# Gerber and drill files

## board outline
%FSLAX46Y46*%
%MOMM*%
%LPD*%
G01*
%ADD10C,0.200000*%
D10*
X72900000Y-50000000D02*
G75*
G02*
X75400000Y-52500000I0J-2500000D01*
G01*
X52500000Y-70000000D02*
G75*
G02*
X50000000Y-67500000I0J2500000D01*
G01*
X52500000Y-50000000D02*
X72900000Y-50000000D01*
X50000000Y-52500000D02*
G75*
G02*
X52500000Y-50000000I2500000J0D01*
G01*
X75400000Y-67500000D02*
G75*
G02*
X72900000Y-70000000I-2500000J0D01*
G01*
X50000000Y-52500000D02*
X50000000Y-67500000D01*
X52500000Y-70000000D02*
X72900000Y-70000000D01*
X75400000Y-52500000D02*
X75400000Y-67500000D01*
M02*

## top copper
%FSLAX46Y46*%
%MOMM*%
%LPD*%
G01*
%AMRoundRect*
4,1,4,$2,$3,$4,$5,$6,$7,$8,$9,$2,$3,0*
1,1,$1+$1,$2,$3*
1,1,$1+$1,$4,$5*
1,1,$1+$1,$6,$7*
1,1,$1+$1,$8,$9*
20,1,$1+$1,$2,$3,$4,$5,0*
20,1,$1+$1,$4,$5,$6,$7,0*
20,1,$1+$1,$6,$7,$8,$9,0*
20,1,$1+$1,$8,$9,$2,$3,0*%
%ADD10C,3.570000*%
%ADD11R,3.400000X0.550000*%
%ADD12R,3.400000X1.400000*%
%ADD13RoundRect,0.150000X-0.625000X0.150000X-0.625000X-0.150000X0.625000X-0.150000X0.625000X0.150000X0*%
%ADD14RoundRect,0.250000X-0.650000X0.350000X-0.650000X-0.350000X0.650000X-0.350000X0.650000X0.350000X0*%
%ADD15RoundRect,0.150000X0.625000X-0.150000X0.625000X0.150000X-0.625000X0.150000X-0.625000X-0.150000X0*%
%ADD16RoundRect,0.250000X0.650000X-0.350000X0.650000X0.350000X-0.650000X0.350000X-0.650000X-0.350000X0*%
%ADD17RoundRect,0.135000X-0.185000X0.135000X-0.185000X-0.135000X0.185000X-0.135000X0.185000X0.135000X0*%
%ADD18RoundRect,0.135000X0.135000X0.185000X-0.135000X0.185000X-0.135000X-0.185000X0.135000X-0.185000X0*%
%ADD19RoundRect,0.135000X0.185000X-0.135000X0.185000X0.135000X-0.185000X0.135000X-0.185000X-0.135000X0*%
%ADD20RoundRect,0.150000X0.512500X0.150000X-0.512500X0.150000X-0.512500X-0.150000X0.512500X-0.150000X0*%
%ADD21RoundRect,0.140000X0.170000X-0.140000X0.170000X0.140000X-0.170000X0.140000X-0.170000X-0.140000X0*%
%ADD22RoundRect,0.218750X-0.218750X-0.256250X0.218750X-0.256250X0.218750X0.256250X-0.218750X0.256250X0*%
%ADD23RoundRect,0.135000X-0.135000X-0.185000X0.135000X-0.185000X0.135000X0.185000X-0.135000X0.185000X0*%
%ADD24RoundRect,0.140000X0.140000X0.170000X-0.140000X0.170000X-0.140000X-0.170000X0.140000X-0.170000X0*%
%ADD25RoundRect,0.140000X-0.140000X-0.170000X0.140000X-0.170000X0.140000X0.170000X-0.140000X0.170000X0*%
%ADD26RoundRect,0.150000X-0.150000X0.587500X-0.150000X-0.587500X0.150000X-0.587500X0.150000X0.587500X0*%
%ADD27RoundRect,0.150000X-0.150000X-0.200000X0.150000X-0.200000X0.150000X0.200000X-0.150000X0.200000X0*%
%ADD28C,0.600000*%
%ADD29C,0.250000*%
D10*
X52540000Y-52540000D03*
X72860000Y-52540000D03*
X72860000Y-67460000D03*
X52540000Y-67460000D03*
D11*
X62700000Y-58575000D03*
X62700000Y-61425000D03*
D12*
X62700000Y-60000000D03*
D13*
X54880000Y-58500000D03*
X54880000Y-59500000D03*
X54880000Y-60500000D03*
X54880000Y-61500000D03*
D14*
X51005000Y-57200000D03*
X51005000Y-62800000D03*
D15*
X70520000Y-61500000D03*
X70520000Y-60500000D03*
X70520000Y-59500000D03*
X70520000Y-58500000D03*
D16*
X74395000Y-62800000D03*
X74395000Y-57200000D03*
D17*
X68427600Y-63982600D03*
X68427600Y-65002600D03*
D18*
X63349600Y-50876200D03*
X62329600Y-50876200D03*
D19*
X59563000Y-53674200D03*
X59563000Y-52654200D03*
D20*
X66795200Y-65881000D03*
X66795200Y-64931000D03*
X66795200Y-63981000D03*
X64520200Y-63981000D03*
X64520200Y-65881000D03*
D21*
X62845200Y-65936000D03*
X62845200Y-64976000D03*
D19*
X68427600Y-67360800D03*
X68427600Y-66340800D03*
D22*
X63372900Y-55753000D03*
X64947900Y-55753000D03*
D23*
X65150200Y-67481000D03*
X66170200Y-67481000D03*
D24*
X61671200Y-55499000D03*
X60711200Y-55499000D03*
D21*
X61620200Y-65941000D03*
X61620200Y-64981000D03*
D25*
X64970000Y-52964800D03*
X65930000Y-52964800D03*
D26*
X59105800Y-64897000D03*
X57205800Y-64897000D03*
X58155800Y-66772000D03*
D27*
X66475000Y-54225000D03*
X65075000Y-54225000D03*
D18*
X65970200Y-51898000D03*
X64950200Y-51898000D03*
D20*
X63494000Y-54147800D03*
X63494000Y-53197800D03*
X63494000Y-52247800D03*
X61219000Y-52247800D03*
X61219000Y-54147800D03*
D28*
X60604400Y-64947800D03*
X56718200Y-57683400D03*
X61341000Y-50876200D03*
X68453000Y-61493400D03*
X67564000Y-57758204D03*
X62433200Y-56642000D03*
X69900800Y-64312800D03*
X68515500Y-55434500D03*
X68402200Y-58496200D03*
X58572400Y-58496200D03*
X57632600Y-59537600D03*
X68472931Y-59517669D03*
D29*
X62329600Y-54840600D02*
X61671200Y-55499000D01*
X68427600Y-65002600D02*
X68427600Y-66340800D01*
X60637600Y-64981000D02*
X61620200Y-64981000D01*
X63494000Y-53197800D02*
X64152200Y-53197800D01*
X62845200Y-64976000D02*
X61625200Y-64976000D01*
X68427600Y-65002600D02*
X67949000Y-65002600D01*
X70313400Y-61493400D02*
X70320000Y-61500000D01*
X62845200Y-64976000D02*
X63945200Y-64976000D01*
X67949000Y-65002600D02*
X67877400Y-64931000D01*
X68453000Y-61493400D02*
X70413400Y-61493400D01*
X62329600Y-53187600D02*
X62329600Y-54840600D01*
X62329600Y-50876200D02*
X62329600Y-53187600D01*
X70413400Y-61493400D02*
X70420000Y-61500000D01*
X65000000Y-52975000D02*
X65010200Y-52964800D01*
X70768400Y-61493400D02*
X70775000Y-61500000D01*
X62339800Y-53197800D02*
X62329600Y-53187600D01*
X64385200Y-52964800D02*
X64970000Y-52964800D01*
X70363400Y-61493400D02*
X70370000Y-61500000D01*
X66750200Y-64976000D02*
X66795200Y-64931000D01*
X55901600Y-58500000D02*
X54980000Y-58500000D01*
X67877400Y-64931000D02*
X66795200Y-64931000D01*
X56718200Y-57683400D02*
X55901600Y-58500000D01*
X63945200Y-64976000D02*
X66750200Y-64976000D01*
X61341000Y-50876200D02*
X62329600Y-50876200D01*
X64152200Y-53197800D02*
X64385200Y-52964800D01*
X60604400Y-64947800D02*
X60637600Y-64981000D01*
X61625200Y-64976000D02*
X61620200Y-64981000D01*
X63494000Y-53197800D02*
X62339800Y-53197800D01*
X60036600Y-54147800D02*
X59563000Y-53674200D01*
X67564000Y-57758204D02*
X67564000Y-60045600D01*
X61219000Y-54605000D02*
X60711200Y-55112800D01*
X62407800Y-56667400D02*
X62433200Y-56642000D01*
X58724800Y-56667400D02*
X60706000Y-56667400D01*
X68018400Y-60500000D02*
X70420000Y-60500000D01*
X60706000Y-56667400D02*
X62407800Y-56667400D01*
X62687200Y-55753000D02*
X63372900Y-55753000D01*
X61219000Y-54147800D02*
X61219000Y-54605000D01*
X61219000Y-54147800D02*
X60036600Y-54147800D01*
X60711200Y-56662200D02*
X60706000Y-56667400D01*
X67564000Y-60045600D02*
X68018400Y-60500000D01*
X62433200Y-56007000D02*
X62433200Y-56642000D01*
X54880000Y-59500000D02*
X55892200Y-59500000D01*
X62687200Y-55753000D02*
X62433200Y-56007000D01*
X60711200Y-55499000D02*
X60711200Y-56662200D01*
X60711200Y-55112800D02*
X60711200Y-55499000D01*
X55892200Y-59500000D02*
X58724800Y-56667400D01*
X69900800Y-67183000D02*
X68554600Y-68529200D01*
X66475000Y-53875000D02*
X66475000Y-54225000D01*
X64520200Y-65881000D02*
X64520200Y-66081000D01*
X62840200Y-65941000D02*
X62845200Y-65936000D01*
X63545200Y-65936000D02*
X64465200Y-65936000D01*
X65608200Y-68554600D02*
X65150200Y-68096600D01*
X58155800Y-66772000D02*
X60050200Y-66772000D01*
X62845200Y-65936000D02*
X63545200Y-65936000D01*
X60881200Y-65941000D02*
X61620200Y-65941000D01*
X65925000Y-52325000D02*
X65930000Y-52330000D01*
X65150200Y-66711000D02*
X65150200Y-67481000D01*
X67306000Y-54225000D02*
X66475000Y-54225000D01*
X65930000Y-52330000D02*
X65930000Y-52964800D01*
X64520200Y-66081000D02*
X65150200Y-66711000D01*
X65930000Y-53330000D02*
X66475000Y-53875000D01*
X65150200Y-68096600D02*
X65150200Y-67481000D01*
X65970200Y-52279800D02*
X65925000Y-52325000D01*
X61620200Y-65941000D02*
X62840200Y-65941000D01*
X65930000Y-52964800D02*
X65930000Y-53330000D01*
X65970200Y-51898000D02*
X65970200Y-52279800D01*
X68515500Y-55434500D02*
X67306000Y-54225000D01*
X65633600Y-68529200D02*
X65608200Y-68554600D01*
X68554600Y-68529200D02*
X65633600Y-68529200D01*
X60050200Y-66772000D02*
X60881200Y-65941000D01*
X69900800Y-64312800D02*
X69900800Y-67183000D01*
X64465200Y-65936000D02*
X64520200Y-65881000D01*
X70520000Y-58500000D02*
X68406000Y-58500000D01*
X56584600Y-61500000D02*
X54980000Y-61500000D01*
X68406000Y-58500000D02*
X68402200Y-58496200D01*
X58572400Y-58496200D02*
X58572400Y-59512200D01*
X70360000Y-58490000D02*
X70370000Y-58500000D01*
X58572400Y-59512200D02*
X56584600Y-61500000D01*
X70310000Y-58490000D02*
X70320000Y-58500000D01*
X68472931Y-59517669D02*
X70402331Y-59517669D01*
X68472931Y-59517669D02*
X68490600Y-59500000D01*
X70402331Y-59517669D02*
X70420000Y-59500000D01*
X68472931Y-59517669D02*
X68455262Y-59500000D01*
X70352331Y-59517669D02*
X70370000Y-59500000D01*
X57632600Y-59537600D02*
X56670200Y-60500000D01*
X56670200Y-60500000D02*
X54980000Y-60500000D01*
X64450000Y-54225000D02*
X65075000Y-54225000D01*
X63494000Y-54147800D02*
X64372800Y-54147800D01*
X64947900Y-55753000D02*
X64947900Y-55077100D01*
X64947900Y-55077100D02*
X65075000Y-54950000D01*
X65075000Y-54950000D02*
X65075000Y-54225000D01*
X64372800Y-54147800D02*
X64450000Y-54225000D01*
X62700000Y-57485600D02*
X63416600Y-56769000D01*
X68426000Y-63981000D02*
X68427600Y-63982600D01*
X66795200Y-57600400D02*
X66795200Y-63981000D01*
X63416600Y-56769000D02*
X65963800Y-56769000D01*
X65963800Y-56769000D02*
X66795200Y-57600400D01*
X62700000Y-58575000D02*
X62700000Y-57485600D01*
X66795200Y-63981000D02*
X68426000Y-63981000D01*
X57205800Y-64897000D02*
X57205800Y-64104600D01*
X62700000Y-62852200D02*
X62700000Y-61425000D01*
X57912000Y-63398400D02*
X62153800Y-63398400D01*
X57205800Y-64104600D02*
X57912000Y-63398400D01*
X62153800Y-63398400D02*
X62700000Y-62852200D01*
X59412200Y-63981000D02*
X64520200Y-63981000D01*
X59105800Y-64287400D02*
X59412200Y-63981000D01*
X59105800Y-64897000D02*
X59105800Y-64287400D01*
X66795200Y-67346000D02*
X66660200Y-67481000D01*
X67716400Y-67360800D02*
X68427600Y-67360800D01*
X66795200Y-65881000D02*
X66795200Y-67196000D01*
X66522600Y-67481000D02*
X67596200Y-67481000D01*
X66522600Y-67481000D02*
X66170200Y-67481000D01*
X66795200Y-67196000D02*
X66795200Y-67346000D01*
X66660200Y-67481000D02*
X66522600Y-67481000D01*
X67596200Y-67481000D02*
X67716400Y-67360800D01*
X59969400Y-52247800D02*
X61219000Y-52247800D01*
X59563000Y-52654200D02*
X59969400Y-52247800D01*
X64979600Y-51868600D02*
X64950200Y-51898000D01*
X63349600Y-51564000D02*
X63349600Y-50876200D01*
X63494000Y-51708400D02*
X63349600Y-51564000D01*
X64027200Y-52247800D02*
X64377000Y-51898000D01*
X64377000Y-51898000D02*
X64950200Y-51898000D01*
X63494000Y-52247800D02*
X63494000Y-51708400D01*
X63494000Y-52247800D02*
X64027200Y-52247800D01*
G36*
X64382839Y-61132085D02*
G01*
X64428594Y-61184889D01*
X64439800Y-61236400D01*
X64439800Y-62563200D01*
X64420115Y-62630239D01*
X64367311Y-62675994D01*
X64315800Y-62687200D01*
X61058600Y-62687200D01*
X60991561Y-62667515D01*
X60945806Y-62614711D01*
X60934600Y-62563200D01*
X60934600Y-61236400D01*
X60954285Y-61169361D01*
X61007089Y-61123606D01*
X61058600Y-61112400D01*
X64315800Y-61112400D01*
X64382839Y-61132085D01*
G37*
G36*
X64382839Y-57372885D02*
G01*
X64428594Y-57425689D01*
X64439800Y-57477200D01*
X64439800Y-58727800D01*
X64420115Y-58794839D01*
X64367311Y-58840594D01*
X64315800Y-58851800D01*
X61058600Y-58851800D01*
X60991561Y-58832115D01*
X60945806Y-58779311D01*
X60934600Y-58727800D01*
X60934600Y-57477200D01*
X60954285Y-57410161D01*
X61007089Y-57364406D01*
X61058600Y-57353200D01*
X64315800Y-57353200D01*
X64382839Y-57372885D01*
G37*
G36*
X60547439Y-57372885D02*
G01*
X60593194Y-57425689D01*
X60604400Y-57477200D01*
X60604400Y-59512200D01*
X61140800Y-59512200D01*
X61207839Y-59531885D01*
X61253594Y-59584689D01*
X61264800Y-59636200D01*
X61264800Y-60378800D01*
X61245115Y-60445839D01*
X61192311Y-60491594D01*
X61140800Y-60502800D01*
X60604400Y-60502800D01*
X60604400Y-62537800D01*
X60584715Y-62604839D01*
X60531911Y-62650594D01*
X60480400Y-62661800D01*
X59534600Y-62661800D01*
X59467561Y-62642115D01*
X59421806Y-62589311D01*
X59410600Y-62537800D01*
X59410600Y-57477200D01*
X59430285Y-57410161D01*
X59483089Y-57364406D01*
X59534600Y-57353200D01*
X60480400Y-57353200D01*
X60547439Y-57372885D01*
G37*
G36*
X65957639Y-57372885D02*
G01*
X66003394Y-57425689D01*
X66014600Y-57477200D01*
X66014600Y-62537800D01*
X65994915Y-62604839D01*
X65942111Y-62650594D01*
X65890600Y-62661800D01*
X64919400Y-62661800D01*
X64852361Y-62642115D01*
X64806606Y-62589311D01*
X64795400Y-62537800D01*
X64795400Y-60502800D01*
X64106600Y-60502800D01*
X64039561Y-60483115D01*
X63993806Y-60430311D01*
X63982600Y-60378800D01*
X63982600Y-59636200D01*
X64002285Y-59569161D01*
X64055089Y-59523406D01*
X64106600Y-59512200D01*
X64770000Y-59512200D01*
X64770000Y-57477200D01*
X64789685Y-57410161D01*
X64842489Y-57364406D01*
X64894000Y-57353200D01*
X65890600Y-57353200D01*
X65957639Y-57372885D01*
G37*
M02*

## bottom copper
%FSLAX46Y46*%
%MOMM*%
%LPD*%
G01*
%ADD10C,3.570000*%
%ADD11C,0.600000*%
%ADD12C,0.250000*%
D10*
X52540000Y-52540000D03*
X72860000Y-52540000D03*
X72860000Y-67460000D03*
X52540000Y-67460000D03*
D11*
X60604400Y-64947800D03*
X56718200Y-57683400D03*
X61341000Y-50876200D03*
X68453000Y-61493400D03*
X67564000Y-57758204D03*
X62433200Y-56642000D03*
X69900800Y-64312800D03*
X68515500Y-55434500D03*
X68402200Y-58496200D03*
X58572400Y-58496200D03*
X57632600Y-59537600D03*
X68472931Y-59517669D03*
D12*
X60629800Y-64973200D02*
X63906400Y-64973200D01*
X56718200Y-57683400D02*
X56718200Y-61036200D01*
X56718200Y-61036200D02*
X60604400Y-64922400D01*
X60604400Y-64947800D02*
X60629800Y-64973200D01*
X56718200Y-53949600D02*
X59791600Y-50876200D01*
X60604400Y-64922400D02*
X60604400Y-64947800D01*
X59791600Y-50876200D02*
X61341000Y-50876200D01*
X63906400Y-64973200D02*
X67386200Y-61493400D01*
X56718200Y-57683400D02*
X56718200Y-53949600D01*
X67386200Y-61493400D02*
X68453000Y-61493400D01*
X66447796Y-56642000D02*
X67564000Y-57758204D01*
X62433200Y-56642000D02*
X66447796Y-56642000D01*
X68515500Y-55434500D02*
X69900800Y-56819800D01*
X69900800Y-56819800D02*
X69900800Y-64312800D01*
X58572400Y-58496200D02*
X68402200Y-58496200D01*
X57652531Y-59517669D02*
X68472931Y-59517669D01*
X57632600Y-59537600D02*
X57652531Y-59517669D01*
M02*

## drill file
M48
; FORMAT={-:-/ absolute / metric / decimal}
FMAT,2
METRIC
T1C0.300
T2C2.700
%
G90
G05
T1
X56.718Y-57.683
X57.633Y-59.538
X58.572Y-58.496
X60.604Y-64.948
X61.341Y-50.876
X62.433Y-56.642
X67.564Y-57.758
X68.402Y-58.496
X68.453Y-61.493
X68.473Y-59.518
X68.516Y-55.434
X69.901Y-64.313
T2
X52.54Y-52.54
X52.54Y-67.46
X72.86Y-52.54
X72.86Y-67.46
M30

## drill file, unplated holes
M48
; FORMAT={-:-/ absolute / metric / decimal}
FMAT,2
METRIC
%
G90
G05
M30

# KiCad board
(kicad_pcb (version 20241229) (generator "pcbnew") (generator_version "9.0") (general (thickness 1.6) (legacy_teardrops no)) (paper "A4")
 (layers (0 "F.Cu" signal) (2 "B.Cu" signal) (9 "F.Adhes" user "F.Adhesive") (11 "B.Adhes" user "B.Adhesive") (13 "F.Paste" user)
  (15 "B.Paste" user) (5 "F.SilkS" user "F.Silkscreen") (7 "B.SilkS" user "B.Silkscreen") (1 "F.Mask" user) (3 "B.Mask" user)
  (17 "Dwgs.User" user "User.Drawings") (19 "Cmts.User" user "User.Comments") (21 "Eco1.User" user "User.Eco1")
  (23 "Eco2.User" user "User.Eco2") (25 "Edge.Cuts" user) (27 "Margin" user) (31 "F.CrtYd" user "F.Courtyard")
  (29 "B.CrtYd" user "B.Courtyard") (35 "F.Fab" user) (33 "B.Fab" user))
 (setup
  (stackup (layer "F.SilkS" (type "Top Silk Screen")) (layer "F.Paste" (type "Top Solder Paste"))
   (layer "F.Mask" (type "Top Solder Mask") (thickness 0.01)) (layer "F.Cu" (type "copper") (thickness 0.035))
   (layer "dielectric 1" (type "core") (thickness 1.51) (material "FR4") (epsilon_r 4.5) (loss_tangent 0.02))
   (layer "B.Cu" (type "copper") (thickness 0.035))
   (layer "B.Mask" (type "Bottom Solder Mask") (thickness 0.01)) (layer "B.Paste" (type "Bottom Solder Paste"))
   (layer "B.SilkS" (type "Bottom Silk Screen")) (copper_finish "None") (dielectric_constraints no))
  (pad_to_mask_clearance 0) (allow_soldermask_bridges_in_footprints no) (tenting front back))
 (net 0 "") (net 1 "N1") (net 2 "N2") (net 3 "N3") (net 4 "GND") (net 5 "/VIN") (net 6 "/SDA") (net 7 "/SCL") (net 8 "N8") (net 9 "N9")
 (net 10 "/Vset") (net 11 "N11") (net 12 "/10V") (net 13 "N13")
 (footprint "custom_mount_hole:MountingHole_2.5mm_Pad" (layer "F.Cu") (at 52.54 52.54)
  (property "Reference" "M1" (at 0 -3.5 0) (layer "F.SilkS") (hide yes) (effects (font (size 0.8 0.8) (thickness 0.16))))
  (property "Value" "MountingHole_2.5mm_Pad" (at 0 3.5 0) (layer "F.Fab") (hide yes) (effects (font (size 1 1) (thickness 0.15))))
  (pad "~" thru_hole circle (at 0 0) (size 3.57 3.57) (drill 2.7) (layers "*.Cu" "*.Mask") (remove_unused_layers no)))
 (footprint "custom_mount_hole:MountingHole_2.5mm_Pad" (layer "F.Cu") (at 72.86 52.54)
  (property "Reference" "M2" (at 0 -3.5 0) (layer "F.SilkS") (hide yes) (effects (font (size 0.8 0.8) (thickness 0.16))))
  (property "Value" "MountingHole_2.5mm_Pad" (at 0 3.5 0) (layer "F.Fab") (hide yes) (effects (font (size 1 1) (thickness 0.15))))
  (pad "~" thru_hole circle (at 0 0) (size 3.57 3.57) (drill 2.7) (layers "*.Cu" "*.Mask") (remove_unused_layers no)))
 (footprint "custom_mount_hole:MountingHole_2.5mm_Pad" (layer "F.Cu") (at 72.86 67.46)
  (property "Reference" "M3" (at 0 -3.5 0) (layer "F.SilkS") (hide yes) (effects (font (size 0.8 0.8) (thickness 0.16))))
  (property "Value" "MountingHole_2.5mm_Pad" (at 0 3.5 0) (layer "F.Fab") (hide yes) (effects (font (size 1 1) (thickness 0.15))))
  (pad "~" thru_hole circle (at 0 0) (size 3.57 3.57) (drill 2.7) (layers "*.Cu" "*.Mask") (remove_unused_layers no)))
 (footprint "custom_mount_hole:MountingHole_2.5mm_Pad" (layer "F.Cu") (at 52.54 67.46)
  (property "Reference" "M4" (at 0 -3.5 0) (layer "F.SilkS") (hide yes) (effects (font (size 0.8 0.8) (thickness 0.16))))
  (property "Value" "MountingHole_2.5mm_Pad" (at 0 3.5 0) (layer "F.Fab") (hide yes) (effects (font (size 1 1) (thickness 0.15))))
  (pad "~" thru_hole circle (at 0 0) (size 3.57 3.57) (drill 2.7) (layers "*.Cu" "*.Mask") (remove_unused_layers no)))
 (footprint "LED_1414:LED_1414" (layer "F.Cu") (at 62.7 60 -90)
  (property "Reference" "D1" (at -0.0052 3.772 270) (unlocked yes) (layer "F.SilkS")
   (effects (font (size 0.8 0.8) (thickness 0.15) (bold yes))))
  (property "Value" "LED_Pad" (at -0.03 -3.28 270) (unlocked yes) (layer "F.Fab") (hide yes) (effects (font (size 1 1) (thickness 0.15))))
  (pad "1" smd rect (at -1.425 0 270) (size 0.55 3.4) (layers "F.Cu" "F.Mask" "F.Paste") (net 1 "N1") (thermal_bridge_angle 45))
  (pad "2" smd rect (at 1.425 0 270) (size 0.55 3.4) (layers "F.Cu" "F.Mask" "F.Paste") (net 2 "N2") (thermal_bridge_angle 45))
  (pad "3" smd rect (at 0 0 270) (size 1.4 3.4) (layers "F.Cu" "F.Mask" "F.Paste") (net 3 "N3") (thermal_bridge_angle 45)))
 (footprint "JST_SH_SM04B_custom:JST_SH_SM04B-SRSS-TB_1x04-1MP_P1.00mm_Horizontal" (layer "F.Cu") (at 52.88 60 -90)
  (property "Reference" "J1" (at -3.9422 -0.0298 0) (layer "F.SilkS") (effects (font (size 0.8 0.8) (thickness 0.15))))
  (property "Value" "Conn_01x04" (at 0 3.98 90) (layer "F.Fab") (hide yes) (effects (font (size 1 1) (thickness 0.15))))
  (pad "1" smd roundrect (at -1.5 -2 270) (size 0.6 1.55) (layers "F.Cu" "F.Mask" "F.Paste") (roundrect_rratio 0.25) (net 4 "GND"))
  (pad "2" smd roundrect (at -0.5 -2 270) (size 0.6 1.55) (layers "F.Cu" "F.Mask" "F.Paste") (roundrect_rratio 0.25) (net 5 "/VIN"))
  (pad "3" smd roundrect (at 0.5 -2 270) (size 0.6 1.55) (layers "F.Cu" "F.Mask" "F.Paste") (roundrect_rratio 0.25) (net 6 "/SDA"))
  (pad "4" smd roundrect (at 1.5 -2 270) (size 0.6 1.55) (layers "F.Cu" "F.Mask" "F.Paste") (roundrect_rratio 0.25) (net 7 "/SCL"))
  (pad "MP" smd roundrect (at -2.8 1.875 270) (size 1.2 1.8) (layers "F.Cu" "F.Mask" "F.Paste") (roundrect_rratio 0.2083333333))
  (pad "MP" smd roundrect (at 2.8 1.875 270) (size 1.2 1.8) (layers "F.Cu" "F.Mask" "F.Paste") (roundrect_rratio 0.2083333333)))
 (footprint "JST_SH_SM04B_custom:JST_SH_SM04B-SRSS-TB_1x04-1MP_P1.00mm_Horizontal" (layer "F.Cu") (at 72.52 60 90)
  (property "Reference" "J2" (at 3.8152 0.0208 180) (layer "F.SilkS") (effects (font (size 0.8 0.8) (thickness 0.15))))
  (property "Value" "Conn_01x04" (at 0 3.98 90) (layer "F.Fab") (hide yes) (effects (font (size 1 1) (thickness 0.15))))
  (pad "1" smd roundrect (at -1.5 -2 90) (size 0.6 1.55) (layers "F.Cu" "F.Mask" "F.Paste") (roundrect_rratio 0.25) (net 4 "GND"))
  (pad "2" smd roundrect (at -0.5 -2 90) (size 0.6 1.55) (layers "F.Cu" "F.Mask" "F.Paste") (roundrect_rratio 0.25) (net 5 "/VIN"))
  (pad "3" smd roundrect (at 0.5 -2 90) (size 0.6 1.55) (layers "F.Cu" "F.Mask" "F.Paste") (roundrect_rratio 0.25) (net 6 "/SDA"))
  (pad "4" smd roundrect (at 1.5 -2 90) (size 0.6 1.55) (layers "F.Cu" "F.Mask" "F.Paste") (roundrect_rratio 0.25) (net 7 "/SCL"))
  (pad "MP" smd roundrect (at -2.8 1.875 90) (size 1.2 1.8) (layers "F.Cu" "F.Mask" "F.Paste") (roundrect_rratio 0.2083333333))
  (pad "MP" smd roundrect (at 2.8 1.875 90) (size 1.2 1.8) (layers "F.Cu" "F.Mask" "F.Paste") (roundrect_rratio 0.2083333333)))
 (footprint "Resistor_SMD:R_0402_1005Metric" (layer "F.Cu") (at 68.4276 64.4926 -90)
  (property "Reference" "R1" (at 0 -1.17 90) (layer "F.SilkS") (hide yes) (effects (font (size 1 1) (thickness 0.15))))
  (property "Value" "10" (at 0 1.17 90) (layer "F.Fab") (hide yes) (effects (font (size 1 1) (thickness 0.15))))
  (pad "1" smd roundrect (at -0.51 0 270) (size 0.54 0.64) (layers "F.Cu" "F.Mask" "F.Paste") (roundrect_rratio 0.25) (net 1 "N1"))
  (pad "2" smd roundrect (at 0.51 0 270) (size 0.54 0.64) (layers "F.Cu" "F.Mask" "F.Paste") (roundrect_rratio 0.25) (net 4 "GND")))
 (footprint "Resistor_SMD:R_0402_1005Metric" (layer "F.Cu") (at 62.8396 50.8762 180)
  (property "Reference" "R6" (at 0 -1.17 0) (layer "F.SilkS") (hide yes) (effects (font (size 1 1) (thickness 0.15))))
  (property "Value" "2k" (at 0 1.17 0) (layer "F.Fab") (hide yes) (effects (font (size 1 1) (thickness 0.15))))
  (pad "1" smd roundrect (at -0.51 0 180) (size 0.54 0.64) (layers "F.Cu" "F.Mask" "F.Paste") (roundrect_rratio 0.25) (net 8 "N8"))
  (pad "2" smd roundrect (at 0.51 0 180) (size 0.54 0.64) (layers "F.Cu" "F.Mask" "F.Paste") (roundrect_rratio 0.25) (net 4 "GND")))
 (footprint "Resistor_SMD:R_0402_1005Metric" (layer "F.Cu") (at 59.563 53.1642 90)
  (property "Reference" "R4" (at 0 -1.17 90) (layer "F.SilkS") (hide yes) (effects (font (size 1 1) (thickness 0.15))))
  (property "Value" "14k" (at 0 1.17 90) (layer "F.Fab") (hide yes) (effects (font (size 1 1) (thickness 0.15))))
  (pad "1" smd roundrect (at -0.51 0 90) (size 0.54 0.64) (layers "F.Cu" "F.Mask" "F.Paste") (roundrect_rratio 0.25) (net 5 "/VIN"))
  (pad "2" smd roundrect (at 0.51 0 90) (size 0.54 0.64) (layers "F.Cu" "F.Mask" "F.Paste") (roundrect_rratio 0.25) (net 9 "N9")))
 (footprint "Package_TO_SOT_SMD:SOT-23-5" (layer "F.Cu") (at 65.6577 64.931 180)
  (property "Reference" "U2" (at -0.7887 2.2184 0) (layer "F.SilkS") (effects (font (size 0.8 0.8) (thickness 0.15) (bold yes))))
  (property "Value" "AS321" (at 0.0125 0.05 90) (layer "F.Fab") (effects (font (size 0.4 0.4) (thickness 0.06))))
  (pad "1" smd roundrect (at -1.1375 -0.95 180) (size 1.325 0.6) (layers "F.Cu" "F.Mask" "F.Paste") (roundrect_rratio 0.25) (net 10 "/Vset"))
  (pad "2" smd roundrect (at -1.1375 0 180) (size 1.325 0.6) (layers "F.Cu" "F.Mask" "F.Paste") (roundrect_rratio 0.25) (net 4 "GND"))
  (pad "3" smd roundrect (at -1.1375 0.95 180) (size 1.325 0.6) (layers "F.Cu" "F.Mask" "F.Paste") (roundrect_rratio 0.25) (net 1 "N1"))
  (pad "4" smd roundrect (at 1.1375 0.95 180) (size 1.325 0.6) (layers "F.Cu" "F.Mask" "F.Paste") (roundrect_rratio 0.25) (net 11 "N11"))
  (pad "5" smd roundrect (at 1.1375 -0.95 180) (size 1.325 0.6) (layers "F.Cu" "F.Mask" "F.Paste") (roundrect_rratio 0.25) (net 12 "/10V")))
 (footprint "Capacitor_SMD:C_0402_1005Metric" (layer "F.Cu") (at 62.8452 65.456 90)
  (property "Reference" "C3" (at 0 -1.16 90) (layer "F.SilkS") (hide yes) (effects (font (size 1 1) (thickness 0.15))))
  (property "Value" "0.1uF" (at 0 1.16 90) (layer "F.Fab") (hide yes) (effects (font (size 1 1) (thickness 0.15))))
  (pad "1" smd roundrect (at -0.48 0 90) (size 0.56 0.62) (layers "F.Cu" "F.Mask" "F.Paste") (roundrect_rratio 0.25) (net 12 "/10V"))
  (pad "2" smd roundrect (at 0.48 0 90) (size 0.56 0.62) (layers "F.Cu" "F.Mask" "F.Paste") (roundrect_rratio 0.25) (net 4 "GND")))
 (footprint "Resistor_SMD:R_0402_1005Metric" (layer "F.Cu") (at 68.4276 66.8508 90)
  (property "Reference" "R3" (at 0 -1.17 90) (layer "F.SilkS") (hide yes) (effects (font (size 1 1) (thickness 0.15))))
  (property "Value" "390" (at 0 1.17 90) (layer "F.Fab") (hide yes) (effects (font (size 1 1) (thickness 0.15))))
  (pad "1" smd roundrect (at -0.51 0 90) (size 0.54 0.64) (layers "F.Cu" "F.Mask" "F.Paste") (roundrect_rratio 0.25) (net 10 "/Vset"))
  (pad "2" smd roundrect (at 0.51 0 90) (size 0.54 0.64) (layers "F.Cu" "F.Mask" "F.Paste") (roundrect_rratio 0.25) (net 4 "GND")))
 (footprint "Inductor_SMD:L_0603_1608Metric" (layer "F.Cu") (at 64.1604 55.753)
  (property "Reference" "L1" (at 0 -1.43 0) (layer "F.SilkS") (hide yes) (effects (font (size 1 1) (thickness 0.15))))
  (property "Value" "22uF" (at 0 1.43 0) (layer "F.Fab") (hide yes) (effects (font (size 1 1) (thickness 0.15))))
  (pad "1" smd roundrect (at -0.7875 0) (size 0.875 0.95) (layers "F.Cu" "F.Mask" "F.Paste") (roundrect_rratio 0.25) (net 5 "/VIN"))
  (pad "2" smd roundrect (at 0.7875 0) (size 0.875 0.95) (layers "F.Cu" "F.Mask" "F.Paste") (roundrect_rratio 0.25) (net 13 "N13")))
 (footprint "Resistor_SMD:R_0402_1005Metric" (layer "F.Cu") (at 65.6602 67.481)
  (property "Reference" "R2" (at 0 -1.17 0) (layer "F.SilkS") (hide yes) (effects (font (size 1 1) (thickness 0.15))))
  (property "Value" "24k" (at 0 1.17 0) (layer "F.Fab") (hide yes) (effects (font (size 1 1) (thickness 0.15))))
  (pad "1" smd roundrect (at -0.51 0) (size 0.54 0.64) (layers "F.Cu" "F.Mask" "F.Paste") (roundrect_rratio 0.25) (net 12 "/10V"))
  (pad "2" smd roundrect (at 0.51 0) (size 0.54 0.64) (layers "F.Cu" "F.Mask" "F.Paste") (roundrect_rratio 0.25) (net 10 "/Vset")))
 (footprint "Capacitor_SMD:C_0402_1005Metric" (layer "F.Cu") (at 61.1912 55.499 180)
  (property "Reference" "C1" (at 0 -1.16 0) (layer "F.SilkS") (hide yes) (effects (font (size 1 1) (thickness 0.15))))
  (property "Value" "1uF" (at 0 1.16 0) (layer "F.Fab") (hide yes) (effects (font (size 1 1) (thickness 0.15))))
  (pad "1" smd roundrect (at -0.48 0 180) (size 0.56 0.62) (layers "F.Cu" "F.Mask" "F.Paste") (roundrect_rratio 0.25) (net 4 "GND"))
  (pad "2" smd roundrect (at 0.48 0 180) (size 0.56 0.62) (layers "F.Cu" "F.Mask" "F.Paste") (roundrect_rratio 0.25) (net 5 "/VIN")))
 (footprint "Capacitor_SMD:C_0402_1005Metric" (layer "F.Cu") (at 61.6202 65.461 90)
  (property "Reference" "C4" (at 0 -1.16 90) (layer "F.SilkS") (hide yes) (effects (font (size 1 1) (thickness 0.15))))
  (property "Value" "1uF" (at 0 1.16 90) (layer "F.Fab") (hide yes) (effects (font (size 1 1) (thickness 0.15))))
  (pad "1" smd roundrect (at -0.48 0 90) (size 0.56 0.62) (layers "F.Cu" "F.Mask" "F.Paste") (roundrect_rratio 0.25) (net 12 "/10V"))
  (pad "2" smd roundrect (at 0.48 0 90) (size 0.56 0.62) (layers "F.Cu" "F.Mask" "F.Paste") (roundrect_rratio 0.25) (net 4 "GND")))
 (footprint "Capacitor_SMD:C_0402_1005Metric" (layer "F.Cu") (at 65.45 52.9648)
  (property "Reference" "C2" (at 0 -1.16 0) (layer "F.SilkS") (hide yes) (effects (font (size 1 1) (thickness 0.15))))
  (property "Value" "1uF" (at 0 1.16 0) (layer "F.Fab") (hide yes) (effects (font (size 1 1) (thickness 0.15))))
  (pad "1" smd roundrect (at -0.48 0) (size 0.56 0.62) (layers "F.Cu" "F.Mask" "F.Paste") (roundrect_rratio 0.25) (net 4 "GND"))
  (pad "2" smd roundrect (at 0.48 0) (size 0.56 0.62) (layers "F.Cu" "F.Mask" "F.Paste") (roundrect_rratio 0.25) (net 12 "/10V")))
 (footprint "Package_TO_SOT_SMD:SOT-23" (layer "F.Cu") (at 58.1558 65.8345 -90)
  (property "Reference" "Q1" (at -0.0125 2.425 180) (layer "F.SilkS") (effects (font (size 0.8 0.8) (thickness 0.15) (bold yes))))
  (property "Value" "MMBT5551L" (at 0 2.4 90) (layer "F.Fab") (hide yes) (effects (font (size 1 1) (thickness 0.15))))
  (pad "1" smd roundrect (at -0.9375 -0.95 270) (size 1.475 0.6) (layers "F.Cu" "F.Mask" "F.Paste") (roundrect_rratio 0.25) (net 11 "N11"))
  (pad "2" smd roundrect (at -0.9375 0.95 270) (size 1.475 0.6) (layers "F.Cu" "F.Mask" "F.Paste") (roundrect_rratio 0.25) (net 2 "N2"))
  (pad "3" smd roundrect (at 0.9375 0 270) (size 1.475 0.6) (layers "F.Cu" "F.Mask" "F.Paste") (roundrect_rratio 0.25) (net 12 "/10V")))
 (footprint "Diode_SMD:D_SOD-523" (layer "F.Cu") (at 65.775 54.225 180)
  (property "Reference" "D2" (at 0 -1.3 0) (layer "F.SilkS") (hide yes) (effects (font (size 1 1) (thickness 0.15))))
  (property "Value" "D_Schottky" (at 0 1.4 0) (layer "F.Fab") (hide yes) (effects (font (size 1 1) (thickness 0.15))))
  (pad "1" smd roundrect (at -0.7 0) (size 0.6 0.7) (layers "F.Cu" "F.Mask" "F.Paste") (roundrect_rratio 0.25) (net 12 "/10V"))
  (pad "2" smd roundrect (at 0.7 0) (size 0.6 0.7) (layers "F.Cu" "F.Mask" "F.Paste") (roundrect_rratio 0.25) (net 13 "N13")))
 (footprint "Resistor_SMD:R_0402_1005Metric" (layer "F.Cu") (at 65.4602 51.898 180)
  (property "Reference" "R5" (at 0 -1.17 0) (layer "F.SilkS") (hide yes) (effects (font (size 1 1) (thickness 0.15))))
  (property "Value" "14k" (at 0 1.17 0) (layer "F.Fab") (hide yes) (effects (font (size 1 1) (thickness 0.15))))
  (pad "1" smd roundrect (at -0.51 0 180) (size 0.54 0.64) (layers "F.Cu" "F.Mask" "F.Paste") (roundrect_rratio 0.25) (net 12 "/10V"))
  (pad "2" smd roundrect (at 0.51 0 180) (size 0.54 0.64) (layers "F.Cu" "F.Mask" "F.Paste") (roundrect_rratio 0.25) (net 8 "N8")))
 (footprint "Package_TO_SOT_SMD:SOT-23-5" (layer "F.Cu") (at 62.3565 53.1978 180)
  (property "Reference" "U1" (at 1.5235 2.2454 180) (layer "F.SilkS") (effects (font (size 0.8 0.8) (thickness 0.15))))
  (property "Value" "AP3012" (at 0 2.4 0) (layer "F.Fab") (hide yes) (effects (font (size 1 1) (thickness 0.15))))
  (pad "1" smd roundrect (at -1.1375 -0.95 180) (size 1.325 0.6) (layers "F.Cu" "F.Mask" "F.Paste") (roundrect_rratio 0.25) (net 13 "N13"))
  (pad "2" smd roundrect (at -1.1375 0 180) (size 1.325 0.6) (layers "F.Cu" "F.Mask" "F.Paste") (roundrect_rratio 0.25) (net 4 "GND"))
  (pad "3" smd roundrect (at -1.1375 0.95 180) (size 1.325 0.6) (layers "F.Cu" "F.Mask" "F.Paste") (roundrect_rratio 0.25) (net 8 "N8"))
  (pad "4" smd roundrect (at 1.1375 0.95 180) (size 1.325 0.6) (layers "F.Cu" "F.Mask" "F.Paste") (roundrect_rratio 0.25) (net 9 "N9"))
  (pad "5" smd roundrect (at 1.1375 -0.95 180) (size 1.325 0.6) (layers "F.Cu" "F.Mask" "F.Paste") (roundrect_rratio 0.25) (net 5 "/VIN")))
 (gr_arc (start 72.9 50) (mid 74.667767 50.732233) (end 75.4 52.5) (stroke (width 0.2) (type solid)) (layer "Edge.Cuts"))
 (gr_arc (start 52.5 70) (mid 50.732233 69.267767) (end 50 67.5) (stroke (width 0.2) (type solid)) (layer "Edge.Cuts"))
 (gr_line (start 52.5 50) (end 72.9 50) (stroke (width 0.2) (type solid)) (layer "Edge.Cuts"))
 (gr_arc (start 50 52.5) (mid 50.732233 50.732233) (end 52.5 50) (stroke (width 0.2) (type solid)) (layer "Edge.Cuts"))
 (gr_arc (start 75.4 67.5) (mid 74.667767 69.267767) (end 72.9 70) (stroke (width 0.2) (type solid)) (layer "Edge.Cuts"))
 (gr_line (start 50 52.5) (end 50 67.5) (stroke (width 0.2) (type solid)) (layer "Edge.Cuts"))
 (gr_line (start 52.5 70) (end 72.9 70) (stroke (width 0.2) (type solid)) (layer "Edge.Cuts"))
 (gr_line (start 75.4 52.5) (end 75.4 67.5) (stroke (width 0.2) (type solid)) (layer "Edge.Cuts"))
 (segment (start 62.3296 54.8406) (end 61.6712 55.499) (width 0.25) (layer "F.Cu") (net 4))
 (segment (start 68.4276 65.0026) (end 68.4276 66.3408) (width 0.25) (layer "F.Cu") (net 4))
 (segment (start 60.6376 64.981) (end 61.6202 64.981) (width 0.25) (layer "F.Cu") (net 4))
 (segment (start 63.494 53.1978) (end 64.1522 53.1978) (width 0.25) (layer "F.Cu") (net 4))
 (segment (start 62.8452 64.976) (end 61.6252 64.976) (width 0.25) (layer "F.Cu") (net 4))
 (segment (start 68.4276 65.0026) (end 67.949 65.0026) (width 0.25) (layer "F.Cu") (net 4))
 (segment (start 70.3134 61.4934) (end 70.32 61.5) (width 0.25) (layer "F.Cu") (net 4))
 (segment (start 62.8452 64.976) (end 63.9452 64.976) (width 0.25) (layer "F.Cu") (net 4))
 (segment (start 67.949 65.0026) (end 67.8774 64.931) (width 0.25) (layer "F.Cu") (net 4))
 (segment (start 68.453 61.4934) (end 70.4134 61.4934) (width 0.25) (layer "F.Cu") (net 4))
 (segment (start 62.3296 53.1876) (end 62.3296 54.8406) (width 0.25) (layer "F.Cu") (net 4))
 (segment (start 62.3296 50.8762) (end 62.3296 53.1876) (width 0.25) (layer "F.Cu") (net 4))
 (segment (start 70.4134 61.4934) (end 70.42 61.5) (width 0.25) (layer "F.Cu") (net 4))
 (segment (start 65 52.975) (end 65.0102 52.9648) (width 0.25) (layer "F.Cu") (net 4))
 (segment (start 70.7684 61.4934) (end 70.775 61.5) (width 0.25) (layer "F.Cu") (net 4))
 (segment (start 62.3398 53.1978) (end 62.3296 53.1876) (width 0.25) (layer "F.Cu") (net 4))
 (segment (start 64.3852 52.9648) (end 64.97 52.9648) (width 0.25) (layer "F.Cu") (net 4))
 (segment (start 70.3634 61.4934) (end 70.37 61.5) (width 0.25) (layer "F.Cu") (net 4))
 (segment (start 66.7502 64.976) (end 66.7952 64.931) (width 0.25) (layer "F.Cu") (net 4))
 (segment (start 55.9016 58.5) (end 54.98 58.5) (width 0.25) (layer "F.Cu") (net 4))
 (segment (start 67.8774 64.931) (end 66.7952 64.931) (width 0.25) (layer "F.Cu") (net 4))
 (segment (start 56.7182 57.6834) (end 55.9016 58.5) (width 0.25) (layer "F.Cu") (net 4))
 (segment (start 63.9452 64.976) (end 66.7502 64.976) (width 0.25) (layer "F.Cu") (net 4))
 (segment (start 61.341 50.8762) (end 62.3296 50.8762) (width 0.25) (layer "F.Cu") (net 4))
 (segment (start 64.1522 53.1978) (end 64.3852 52.9648) (width 0.25) (layer "F.Cu") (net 4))
 (segment (start 60.6044 64.9478) (end 60.6376 64.981) (width 0.25) (layer "F.Cu") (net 4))
 (segment (start 61.6252 64.976) (end 61.6202 64.981) (width 0.25) (layer "F.Cu") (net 4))
 (segment (start 63.494 53.1978) (end 62.3398 53.1978) (width 0.25) (layer "F.Cu") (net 4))
 (via (at 60.6044 64.9478) (size 0.6) (drill 0.3) (layers "F.Cu" "B.Cu") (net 4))
 (via (at 56.7182 57.6834) (size 0.6) (drill 0.3) (layers "F.Cu" "B.Cu") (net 4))
 (via (at 61.341 50.8762) (size 0.6) (drill 0.3) (layers "F.Cu" "B.Cu") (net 4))
 (via (at 68.453 61.4934) (size 0.6) (drill 0.3) (layers "F.Cu" "B.Cu") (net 4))
 (segment (start 60.6298 64.9732) (end 63.9064 64.9732) (width 0.25) (layer "B.Cu") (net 4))
 (segment (start 56.7182 57.6834) (end 56.7182 61.0362) (width 0.25) (layer "B.Cu") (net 4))
 (segment (start 56.7182 61.0362) (end 60.6044 64.9224) (width 0.25) (layer "B.Cu") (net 4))
 (segment (start 60.6044 64.9478) (end 60.6298 64.9732) (width 0.25) (layer "B.Cu") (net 4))
 (segment (start 56.7182 53.9496) (end 59.7916 50.8762) (width 0.25) (layer "B.Cu") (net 4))
 (segment (start 60.6044 64.9224) (end 60.6044 64.9478) (width 0.25) (layer "B.Cu") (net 4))
 (segment (start 59.7916 50.8762) (end 61.341 50.8762) (width 0.25) (layer "B.Cu") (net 4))
 (segment (start 63.9064 64.9732) (end 67.3862 61.4934) (width 0.25) (layer "B.Cu") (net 4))
 (segment (start 56.7182 57.6834) (end 56.7182 53.9496) (width 0.25) (layer "B.Cu") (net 4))
 (segment (start 67.3862 61.4934) (end 68.453 61.4934) (width 0.25) (layer "B.Cu") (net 4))
 (segment (start 60.0366 54.1478) (end 59.563 53.6742) (width 0.25) (layer "F.Cu") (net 5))
 (segment (start 67.564 57.758204) (end 67.564 60.0456) (width 0.25) (layer "F.Cu") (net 5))
 (segment (start 61.219 54.605) (end 60.7112 55.1128) (width 0.25) (layer "F.Cu") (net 5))
 (segment (start 62.4078 56.6674) (end 62.4332 56.642) (width 0.25) (layer "F.Cu") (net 5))
 (segment (start 58.7248 56.6674) (end 60.706 56.6674) (width 0.25) (layer "F.Cu") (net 5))
 (segment (start 68.0184 60.5) (end 70.42 60.5) (width 0.25) (layer "F.Cu") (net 5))
 (segment (start 60.706 56.6674) (end 62.4078 56.6674) (width 0.25) (layer "F.Cu") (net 5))
 (segment (start 62.6872 55.753) (end 63.3729 55.753) (width 0.25) (layer "F.Cu") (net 5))
 (segment (start 61.219 54.1478) (end 61.219 54.605) (width 0.25) (layer "F.Cu") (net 5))
 (segment (start 61.219 54.1478) (end 60.0366 54.1478) (width 0.25) (layer "F.Cu") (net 5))
 (segment (start 60.7112 56.6622) (end 60.706 56.6674) (width 0.25) (layer "F.Cu") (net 5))
 (segment (start 67.564 60.0456) (end 68.0184 60.5) (width 0.25) (layer "F.Cu") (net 5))
 (segment (start 62.4332 56.007) (end 62.4332 56.642) (width 0.25) (layer "F.Cu") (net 5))
 (segment (start 54.88 59.5) (end 55.8922 59.5) (width 0.25) (layer "F.Cu") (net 5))
 (segment (start 62.6872 55.753) (end 62.4332 56.007) (width 0.25) (layer "F.Cu") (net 5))
 (segment (start 60.7112 55.499) (end 60.7112 56.6622) (width 0.25) (layer "F.Cu") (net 5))
 (segment (start 60.7112 55.1128) (end 60.7112 55.499) (width 0.25) (layer "F.Cu") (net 5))
 (segment (start 55.8922 59.5) (end 58.7248 56.6674) (width 0.25) (layer "F.Cu") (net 5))
 (via (at 67.564 57.758204) (size 0.6) (drill 0.3) (layers "F.Cu" "B.Cu") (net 5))
 (via (at 62.4332 56.642) (size 0.6) (drill 0.3) (layers "F.Cu" "B.Cu") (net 5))
 (segment (start 66.447796 56.642) (end 67.564 57.758204) (width 0.25) (layer "B.Cu") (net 5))
 (segment (start 62.4332 56.642) (end 66.447796 56.642) (width 0.25) (layer "B.Cu") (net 5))
 (segment (start 69.9008 67.183) (end 68.5546 68.5292) (width 0.25) (layer "F.Cu") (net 12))
 (segment (start 66.475 53.875) (end 66.475 54.225) (width 0.25) (layer "F.Cu") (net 12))
 (segment (start 64.5202 65.881) (end 64.5202 66.081) (width 0.25) (layer "F.Cu") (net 12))
 (segment (start 62.8402 65.941) (end 62.8452 65.936) (width 0.25) (layer "F.Cu") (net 12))
 (segment (start 63.5452 65.936) (end 64.4652 65.936) (width 0.25) (layer "F.Cu") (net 12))
 (segment (start 65.6082 68.5546) (end 65.1502 68.0966) (width 0.25) (layer "F.Cu") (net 12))
 (segment (start 58.1558 66.772) (end 60.0502 66.772) (width 0.25) (layer "F.Cu") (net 12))
 (segment (start 62.8452 65.936) (end 63.5452 65.936) (width 0.25) (layer "F.Cu") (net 12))
 (segment (start 60.8812 65.941) (end 61.6202 65.941) (width 0.25) (layer "F.Cu") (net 12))
 (segment (start 65.925 52.325) (end 65.93 52.33) (width 0.25) (layer "F.Cu") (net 12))
 (segment (start 65.1502 66.711) (end 65.1502 67.481) (width 0.25) (layer "F.Cu") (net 12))
 (segment (start 67.306 54.225) (end 66.475 54.225) (width 0.25) (layer "F.Cu") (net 12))
 (segment (start 65.93 52.33) (end 65.93 52.9648) (width 0.25) (layer "F.Cu") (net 12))
 (segment (start 64.5202 66.081) (end 65.1502 66.711) (width 0.25) (layer "F.Cu") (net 12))
 (segment (start 65.93 53.33) (end 66.475 53.875) (width 0.25) (layer "F.Cu") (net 12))
 (segment (start 65.1502 68.0966) (end 65.1502 67.481) (width 0.25) (layer "F.Cu") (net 12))
 (segment (start 65.9702 52.2798) (end 65.925 52.325) (width 0.25) (layer "F.Cu") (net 12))
 (segment (start 61.6202 65.941) (end 62.8402 65.941) (width 0.25) (layer "F.Cu") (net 12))
 (segment (start 65.93 52.9648) (end 65.93 53.33) (width 0.25) (layer "F.Cu") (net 12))
 (segment (start 65.9702 51.898) (end 65.9702 52.2798) (width 0.25) (layer "F.Cu") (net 12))
 (segment (start 68.5155 55.4345) (end 67.306 54.225) (width 0.25) (layer "F.Cu") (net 12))
 (segment (start 65.6336 68.5292) (end 65.6082 68.5546) (width 0.25) (layer "F.Cu") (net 12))
 (segment (start 68.5546 68.5292) (end 65.6336 68.5292) (width 0.25) (layer "F.Cu") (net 12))
 (segment (start 60.0502 66.772) (end 60.8812 65.941) (width 0.25) (layer "F.Cu") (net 12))
 (segment (start 69.9008 64.3128) (end 69.9008 67.183) (width 0.25) (layer "F.Cu") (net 12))
 (segment (start 64.4652 65.936) (end 64.5202 65.881) (width 0.25) (layer "F.Cu") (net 12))
 (via (at 69.9008 64.3128) (size 0.6) (drill 0.3) (layers "F.Cu" "B.Cu") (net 12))
 (via (at 68.5155 55.4345) (size 0.6) (drill 0.3) (layers "F.Cu" "B.Cu") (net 12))
 (segment (start 68.5155 55.4345) (end 69.9008 56.8198) (width 0.25) (layer "B.Cu") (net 12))
 (segment (start 69.9008 56.8198) (end 69.9008 64.3128) (width 0.25) (layer "B.Cu") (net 12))
 (segment (start 70.52 58.5) (end 68.406 58.5) (width 0.25) (layer "F.Cu") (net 7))
 (segment (start 56.5846 61.5) (end 54.98 61.5) (width 0.25) (layer "F.Cu") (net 7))
 (segment (start 68.406 58.5) (end 68.4022 58.4962) (width 0.25) (layer "F.Cu") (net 7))
 (segment (start 58.5724 58.4962) (end 58.5724 59.5122) (width 0.25) (layer "F.Cu") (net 7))
 (segment (start 70.36 58.49) (end 70.37 58.5) (width 0.25) (layer "F.Cu") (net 7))
 (segment (start 58.5724 59.5122) (end 56.5846 61.5) (width 0.25) (layer "F.Cu") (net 7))
 (segment (start 70.31 58.49) (end 70.32 58.5) (width 0.25) (layer "F.Cu") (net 7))
 (via (at 68.4022 58.4962) (size 0.6) (drill 0.3) (layers "F.Cu" "B.Cu") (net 7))
 (via (at 58.5724 58.4962) (size 0.6) (drill 0.3) (layers "F.Cu" "B.Cu") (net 7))
 (segment (start 58.5724 58.4962) (end 68.4022 58.4962) (width 0.25) (layer "B.Cu") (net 7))
 (segment (start 68.472931 59.517669) (end 70.402331 59.517669) (width 0.25) (layer "F.Cu") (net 6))
 (segment (start 68.472931 59.517669) (end 68.4906 59.5) (width 0.25) (layer "F.Cu") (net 6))
 (segment (start 70.402331 59.517669) (end 70.42 59.5) (width 0.25) (layer "F.Cu") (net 6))
 (segment (start 68.472931 59.517669) (end 68.455262 59.5) (width 0.25) (layer "F.Cu") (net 6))
 (segment (start 70.352331 59.517669) (end 70.37 59.5) (width 0.25) (layer "F.Cu") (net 6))
 (segment (start 57.6326 59.5376) (end 56.6702 60.5) (width 0.25) (layer "F.Cu") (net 6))
 (segment (start 56.6702 60.5) (end 54.98 60.5) (width 0.25) (layer "F.Cu") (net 6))
 (via (at 57.6326 59.5376) (size 0.6) (drill 0.3) (layers "F.Cu" "B.Cu") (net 6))
 (via (at 68.472931 59.517669) (size 0.6) (drill 0.3) (layers "F.Cu" "B.Cu") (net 6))
 (segment (start 57.652531 59.517669) (end 68.472931 59.517669) (width 0.25) (layer "B.Cu") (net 6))
 (segment (start 57.6326 59.5376) (end 57.652531 59.517669) (width 0.25) (layer "B.Cu") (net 6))
 (segment (start 64.45 54.225) (end 65.075 54.225) (width 0.25) (layer "F.Cu") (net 13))
 (segment (start 63.494 54.1478) (end 64.3728 54.1478) (width 0.25) (layer "F.Cu") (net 13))
 (segment (start 64.9479 55.753) (end 64.9479 55.0771) (width 0.25) (layer "F.Cu") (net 13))
 (segment (start 64.9479 55.0771) (end 65.075 54.95) (width 0.25) (layer "F.Cu") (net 13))
 (segment (start 65.075 54.95) (end 65.075 54.225) (width 0.25) (layer "F.Cu") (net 13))
 (segment (start 64.3728 54.1478) (end 64.45 54.225) (width 0.25) (layer "F.Cu") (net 13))
 (segment (start 62.7 57.4856) (end 63.4166 56.769) (width 0.25) (layer "F.Cu") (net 1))
 (segment (start 68.426 63.981) (end 68.4276 63.9826) (width 0.25) (layer "F.Cu") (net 1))
 (segment (start 66.7952 57.6004) (end 66.7952 63.981) (width 0.25) (layer "F.Cu") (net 1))
 (segment (start 63.4166 56.769) (end 65.9638 56.769) (width 0.25) (layer "F.Cu") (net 1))
 (segment (start 65.9638 56.769) (end 66.7952 57.6004) (width 0.25) (layer "F.Cu") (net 1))
 (segment (start 62.7 58.575) (end 62.7 57.4856) (width 0.25) (layer "F.Cu") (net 1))
 (segment (start 66.7952 63.981) (end 68.426 63.981) (width 0.25) (layer "F.Cu") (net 1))
 (segment (start 57.2058 64.897) (end 57.2058 64.1046) (width 0.25) (layer "F.Cu") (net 2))
 (segment (start 62.7 62.8522) (end 62.7 61.425) (width 0.25) (layer "F.Cu") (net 2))
 (segment (start 57.912 63.3984) (end 62.1538 63.3984) (width 0.25) (layer "F.Cu") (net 2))
 (segment (start 57.2058 64.1046) (end 57.912 63.3984) (width 0.25) (layer "F.Cu") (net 2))
 (segment (start 62.1538 63.3984) (end 62.7 62.8522) (width 0.25) (layer "F.Cu") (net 2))
 (segment (start 59.4122 63.981) (end 64.5202 63.981) (width 0.25) (layer "F.Cu") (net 11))
 (segment (start 59.1058 64.2874) (end 59.4122 63.981) (width 0.25) (layer "F.Cu") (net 11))
 (segment (start 59.1058 64.897) (end 59.1058 64.2874) (width 0.25) (layer "F.Cu") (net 11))
 (segment (start 66.7952 67.346) (end 66.6602 67.481) (width 0.25) (layer "F.Cu") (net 10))
 (segment (start 67.7164 67.3608) (end 68.4276 67.3608) (width 0.25) (layer "F.Cu") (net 10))
 (segment (start 66.7952 65.881) (end 66.7952 67.196) (width 0.25) (layer "F.Cu") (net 10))
 (segment (start 66.5226 67.481) (end 67.5962 67.481) (width 0.25) (layer "F.Cu") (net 10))
 (segment (start 66.5226 67.481) (end 66.1702 67.481) (width 0.25) (layer "F.Cu") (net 10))
 (segment (start 66.7952 67.196) (end 66.7952 67.346) (width 0.25) (layer "F.Cu") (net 10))
 (segment (start 66.6602 67.481) (end 66.5226 67.481) (width 0.25) (layer "F.Cu") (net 10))
 (segment (start 67.5962 67.481) (end 67.7164 67.3608) (width 0.25) (layer "F.Cu") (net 10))
 (segment (start 59.9694 52.2478) (end 61.219 52.2478) (width 0.25) (layer "F.Cu") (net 9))
 (segment (start 59.563 52.6542) (end 59.9694 52.2478) (width 0.25) (layer "F.Cu") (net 9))
 (segment (start 64.9796 51.8686) (end 64.9502 51.898) (width 0.25) (layer "F.Cu") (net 8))
 (segment (start 63.3496 51.564) (end 63.3496 50.8762) (width 0.25) (layer "F.Cu") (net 8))
 (segment (start 63.494 51.7084) (end 63.3496 51.564) (width 0.25) (layer "F.Cu") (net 8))
 (segment (start 64.0272 52.2478) (end 64.377 51.898) (width 0.25) (layer "F.Cu") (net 8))
 (segment (start 64.377 51.898) (end 64.9502 51.898) (width 0.25) (layer "F.Cu") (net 8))
 (segment (start 63.494 52.2478) (end 63.494 51.7084) (width 0.25) (layer "F.Cu") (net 8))
 (segment (start 63.494 52.2478) (end 64.0272 52.2478) (width 0.25) (layer "F.Cu") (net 8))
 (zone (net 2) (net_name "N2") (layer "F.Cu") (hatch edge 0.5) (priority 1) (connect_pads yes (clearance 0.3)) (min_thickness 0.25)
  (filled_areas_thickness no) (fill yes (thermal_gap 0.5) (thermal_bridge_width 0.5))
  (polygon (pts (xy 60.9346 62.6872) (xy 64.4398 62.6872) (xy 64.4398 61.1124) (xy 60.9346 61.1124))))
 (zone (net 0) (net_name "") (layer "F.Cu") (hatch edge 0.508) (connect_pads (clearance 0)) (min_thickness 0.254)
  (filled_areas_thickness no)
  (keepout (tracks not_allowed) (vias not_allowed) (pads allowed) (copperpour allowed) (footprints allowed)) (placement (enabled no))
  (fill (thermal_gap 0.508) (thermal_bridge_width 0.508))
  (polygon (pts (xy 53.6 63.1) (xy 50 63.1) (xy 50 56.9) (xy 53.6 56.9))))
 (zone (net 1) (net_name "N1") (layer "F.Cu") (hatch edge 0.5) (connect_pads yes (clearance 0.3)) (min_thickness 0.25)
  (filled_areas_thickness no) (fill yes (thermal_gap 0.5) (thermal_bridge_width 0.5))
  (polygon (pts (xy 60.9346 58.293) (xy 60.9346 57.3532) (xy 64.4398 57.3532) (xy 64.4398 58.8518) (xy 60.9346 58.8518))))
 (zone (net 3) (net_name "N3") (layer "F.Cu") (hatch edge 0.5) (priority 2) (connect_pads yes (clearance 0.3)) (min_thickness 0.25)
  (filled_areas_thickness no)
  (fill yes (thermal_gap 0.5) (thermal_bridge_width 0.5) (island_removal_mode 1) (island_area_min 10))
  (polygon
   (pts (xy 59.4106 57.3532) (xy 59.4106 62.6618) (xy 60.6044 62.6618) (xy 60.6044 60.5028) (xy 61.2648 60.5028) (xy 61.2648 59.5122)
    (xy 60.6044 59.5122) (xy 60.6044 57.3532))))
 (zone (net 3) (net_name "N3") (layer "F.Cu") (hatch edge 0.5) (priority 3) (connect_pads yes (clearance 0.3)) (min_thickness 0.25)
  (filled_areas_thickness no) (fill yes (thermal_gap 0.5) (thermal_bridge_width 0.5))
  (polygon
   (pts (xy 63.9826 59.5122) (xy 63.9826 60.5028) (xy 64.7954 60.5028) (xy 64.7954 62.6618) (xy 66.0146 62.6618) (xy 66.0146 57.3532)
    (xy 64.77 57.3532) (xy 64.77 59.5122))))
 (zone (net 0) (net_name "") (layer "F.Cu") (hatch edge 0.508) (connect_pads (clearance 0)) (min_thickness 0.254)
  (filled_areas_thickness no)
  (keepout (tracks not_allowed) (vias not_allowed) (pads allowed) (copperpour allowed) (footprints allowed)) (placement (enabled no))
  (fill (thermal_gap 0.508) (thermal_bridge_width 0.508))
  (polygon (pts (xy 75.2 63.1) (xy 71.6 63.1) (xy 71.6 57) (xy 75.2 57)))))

